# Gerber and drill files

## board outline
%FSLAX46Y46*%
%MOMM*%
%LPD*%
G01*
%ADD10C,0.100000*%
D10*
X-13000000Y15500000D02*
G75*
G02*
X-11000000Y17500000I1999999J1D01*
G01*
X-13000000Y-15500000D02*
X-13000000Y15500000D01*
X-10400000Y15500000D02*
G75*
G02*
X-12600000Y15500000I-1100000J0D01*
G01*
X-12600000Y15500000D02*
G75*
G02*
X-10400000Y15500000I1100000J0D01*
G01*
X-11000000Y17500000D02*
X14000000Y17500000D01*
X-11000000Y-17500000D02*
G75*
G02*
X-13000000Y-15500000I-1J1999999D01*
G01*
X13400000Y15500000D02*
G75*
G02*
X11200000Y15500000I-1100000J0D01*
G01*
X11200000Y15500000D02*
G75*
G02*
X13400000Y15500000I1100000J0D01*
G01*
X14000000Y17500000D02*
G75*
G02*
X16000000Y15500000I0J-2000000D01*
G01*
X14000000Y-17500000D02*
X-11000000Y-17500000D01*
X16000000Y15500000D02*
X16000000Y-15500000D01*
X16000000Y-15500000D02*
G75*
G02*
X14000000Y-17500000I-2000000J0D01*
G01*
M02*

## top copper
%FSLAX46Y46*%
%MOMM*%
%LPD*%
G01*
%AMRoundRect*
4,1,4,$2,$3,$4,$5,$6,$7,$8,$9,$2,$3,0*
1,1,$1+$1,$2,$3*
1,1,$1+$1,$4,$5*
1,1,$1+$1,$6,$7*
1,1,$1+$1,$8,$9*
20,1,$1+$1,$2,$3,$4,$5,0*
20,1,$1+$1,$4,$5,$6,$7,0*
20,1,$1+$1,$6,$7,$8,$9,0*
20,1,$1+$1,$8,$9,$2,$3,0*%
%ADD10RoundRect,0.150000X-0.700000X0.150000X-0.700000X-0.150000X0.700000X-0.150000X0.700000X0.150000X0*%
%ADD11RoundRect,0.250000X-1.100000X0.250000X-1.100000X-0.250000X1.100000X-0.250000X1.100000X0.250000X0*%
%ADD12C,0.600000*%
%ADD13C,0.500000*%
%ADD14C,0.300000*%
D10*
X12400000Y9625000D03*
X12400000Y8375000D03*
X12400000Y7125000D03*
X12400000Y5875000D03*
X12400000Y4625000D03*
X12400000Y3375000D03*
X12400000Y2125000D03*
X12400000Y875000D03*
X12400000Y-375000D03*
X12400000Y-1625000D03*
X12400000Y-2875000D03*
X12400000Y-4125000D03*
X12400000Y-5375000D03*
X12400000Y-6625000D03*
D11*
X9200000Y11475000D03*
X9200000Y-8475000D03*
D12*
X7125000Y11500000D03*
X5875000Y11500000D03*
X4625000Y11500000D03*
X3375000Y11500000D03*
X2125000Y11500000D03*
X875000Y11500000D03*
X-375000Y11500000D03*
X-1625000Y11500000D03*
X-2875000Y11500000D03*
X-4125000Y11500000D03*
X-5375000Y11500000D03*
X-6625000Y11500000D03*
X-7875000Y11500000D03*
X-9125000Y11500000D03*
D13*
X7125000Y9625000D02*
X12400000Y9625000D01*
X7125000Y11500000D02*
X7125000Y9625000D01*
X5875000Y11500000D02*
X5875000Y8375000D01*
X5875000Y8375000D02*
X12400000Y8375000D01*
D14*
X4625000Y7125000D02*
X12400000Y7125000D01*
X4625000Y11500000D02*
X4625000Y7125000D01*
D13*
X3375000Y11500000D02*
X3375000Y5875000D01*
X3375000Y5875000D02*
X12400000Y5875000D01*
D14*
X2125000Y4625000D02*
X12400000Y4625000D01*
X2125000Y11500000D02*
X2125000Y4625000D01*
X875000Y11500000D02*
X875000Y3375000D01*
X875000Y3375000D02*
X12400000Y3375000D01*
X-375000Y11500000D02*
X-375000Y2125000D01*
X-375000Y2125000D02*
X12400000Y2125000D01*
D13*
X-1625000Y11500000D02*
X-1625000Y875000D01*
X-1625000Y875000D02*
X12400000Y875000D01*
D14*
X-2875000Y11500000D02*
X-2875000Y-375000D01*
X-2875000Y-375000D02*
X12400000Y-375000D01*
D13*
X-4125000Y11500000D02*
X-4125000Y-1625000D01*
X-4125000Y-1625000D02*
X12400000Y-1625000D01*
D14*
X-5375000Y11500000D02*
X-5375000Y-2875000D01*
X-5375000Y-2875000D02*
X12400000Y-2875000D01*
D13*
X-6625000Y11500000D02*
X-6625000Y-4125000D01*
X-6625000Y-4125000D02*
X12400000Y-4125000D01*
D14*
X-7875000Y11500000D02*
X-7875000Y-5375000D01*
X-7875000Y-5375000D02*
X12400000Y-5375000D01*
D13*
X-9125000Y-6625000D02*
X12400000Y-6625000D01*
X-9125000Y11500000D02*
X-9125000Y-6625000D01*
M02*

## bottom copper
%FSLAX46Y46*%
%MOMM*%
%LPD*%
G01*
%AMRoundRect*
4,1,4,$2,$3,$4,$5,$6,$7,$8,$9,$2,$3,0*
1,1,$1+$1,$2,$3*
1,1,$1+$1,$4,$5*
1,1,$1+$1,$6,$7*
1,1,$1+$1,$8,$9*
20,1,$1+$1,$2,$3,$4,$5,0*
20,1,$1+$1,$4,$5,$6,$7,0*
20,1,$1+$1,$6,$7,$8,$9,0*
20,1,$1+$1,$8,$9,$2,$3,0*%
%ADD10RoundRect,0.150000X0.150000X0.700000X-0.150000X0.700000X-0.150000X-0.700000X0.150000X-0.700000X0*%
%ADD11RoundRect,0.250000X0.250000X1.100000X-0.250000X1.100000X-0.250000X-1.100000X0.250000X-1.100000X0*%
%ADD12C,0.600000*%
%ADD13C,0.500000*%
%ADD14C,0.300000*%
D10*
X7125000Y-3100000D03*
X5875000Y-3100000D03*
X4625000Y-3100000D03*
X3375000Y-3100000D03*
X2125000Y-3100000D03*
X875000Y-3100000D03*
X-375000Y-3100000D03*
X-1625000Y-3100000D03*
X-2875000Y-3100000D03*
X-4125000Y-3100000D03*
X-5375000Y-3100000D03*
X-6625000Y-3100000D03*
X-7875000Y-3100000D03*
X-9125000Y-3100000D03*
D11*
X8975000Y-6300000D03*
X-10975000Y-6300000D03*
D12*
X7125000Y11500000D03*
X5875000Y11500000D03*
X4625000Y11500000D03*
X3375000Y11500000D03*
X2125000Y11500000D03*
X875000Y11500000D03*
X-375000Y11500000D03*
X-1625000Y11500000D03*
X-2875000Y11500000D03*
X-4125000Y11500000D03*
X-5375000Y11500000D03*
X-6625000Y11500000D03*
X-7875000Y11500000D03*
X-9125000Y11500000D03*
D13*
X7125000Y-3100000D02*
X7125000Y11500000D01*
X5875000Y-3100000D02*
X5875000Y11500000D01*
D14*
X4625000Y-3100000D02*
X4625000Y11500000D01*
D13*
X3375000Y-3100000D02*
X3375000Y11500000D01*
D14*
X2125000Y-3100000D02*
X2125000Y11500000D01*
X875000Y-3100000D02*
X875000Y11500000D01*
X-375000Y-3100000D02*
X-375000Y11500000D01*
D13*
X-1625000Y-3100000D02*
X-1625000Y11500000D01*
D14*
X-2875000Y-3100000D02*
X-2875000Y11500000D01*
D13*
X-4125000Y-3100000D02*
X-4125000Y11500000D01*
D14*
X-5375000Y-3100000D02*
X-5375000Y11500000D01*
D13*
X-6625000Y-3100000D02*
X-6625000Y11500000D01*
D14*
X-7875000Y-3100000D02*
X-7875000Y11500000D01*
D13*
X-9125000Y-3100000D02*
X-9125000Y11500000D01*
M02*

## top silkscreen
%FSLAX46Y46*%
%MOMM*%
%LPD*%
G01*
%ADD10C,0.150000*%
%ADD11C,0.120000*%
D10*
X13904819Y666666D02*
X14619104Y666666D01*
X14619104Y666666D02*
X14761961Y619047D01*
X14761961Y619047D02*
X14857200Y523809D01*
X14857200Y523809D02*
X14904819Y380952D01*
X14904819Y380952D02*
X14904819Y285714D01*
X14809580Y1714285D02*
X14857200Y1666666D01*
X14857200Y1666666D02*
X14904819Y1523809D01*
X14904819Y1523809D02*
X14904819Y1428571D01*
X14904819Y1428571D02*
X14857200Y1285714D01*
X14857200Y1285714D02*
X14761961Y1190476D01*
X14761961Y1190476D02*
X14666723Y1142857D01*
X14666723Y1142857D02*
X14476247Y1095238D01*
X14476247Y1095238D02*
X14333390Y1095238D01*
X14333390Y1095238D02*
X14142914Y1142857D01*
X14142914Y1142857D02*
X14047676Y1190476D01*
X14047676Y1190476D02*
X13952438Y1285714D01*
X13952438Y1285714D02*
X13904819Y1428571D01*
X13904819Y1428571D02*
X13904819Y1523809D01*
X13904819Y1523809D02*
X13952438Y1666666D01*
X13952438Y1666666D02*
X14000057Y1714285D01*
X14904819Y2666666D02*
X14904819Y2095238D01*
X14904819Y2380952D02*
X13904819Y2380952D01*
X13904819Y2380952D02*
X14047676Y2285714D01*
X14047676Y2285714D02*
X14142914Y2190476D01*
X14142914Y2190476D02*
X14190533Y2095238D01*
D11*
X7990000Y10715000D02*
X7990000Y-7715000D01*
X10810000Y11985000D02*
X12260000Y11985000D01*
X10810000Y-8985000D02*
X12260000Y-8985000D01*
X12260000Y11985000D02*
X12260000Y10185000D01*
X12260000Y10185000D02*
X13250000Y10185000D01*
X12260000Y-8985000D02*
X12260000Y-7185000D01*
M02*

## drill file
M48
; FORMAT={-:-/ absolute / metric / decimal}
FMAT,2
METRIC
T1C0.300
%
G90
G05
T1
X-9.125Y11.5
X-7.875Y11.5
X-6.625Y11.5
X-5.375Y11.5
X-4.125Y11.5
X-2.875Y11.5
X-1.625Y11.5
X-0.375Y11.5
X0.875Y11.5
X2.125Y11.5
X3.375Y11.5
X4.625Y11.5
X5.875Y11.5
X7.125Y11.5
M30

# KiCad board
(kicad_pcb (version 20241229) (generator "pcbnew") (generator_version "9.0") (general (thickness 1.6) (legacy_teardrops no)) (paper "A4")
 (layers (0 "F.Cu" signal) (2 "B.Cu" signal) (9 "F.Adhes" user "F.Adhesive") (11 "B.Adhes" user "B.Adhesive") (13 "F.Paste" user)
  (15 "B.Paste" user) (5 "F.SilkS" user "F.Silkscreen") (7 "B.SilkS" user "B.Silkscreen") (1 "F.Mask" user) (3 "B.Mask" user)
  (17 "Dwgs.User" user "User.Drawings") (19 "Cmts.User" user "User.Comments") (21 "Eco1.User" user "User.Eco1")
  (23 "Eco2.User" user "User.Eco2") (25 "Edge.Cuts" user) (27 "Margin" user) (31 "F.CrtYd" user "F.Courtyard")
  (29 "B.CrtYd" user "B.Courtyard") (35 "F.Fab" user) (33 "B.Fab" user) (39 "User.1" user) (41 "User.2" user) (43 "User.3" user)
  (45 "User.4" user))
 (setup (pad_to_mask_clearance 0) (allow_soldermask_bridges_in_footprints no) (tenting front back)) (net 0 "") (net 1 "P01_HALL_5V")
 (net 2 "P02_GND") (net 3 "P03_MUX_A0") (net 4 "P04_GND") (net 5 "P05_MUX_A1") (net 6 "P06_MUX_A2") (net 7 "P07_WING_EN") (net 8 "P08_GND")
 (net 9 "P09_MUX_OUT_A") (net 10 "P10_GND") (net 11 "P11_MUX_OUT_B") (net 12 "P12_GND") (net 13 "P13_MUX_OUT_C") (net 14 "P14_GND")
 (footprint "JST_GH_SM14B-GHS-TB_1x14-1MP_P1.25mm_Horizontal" (layer "F.Cu") (at 10.55 -1.5 -90)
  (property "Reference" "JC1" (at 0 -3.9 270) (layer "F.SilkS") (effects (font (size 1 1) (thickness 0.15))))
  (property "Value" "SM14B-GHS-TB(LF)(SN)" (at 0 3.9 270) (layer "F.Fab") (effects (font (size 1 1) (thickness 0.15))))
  (fp_line (start -9.215 2.56) (end 9.215 2.56) (stroke (width 0.12) (type solid)) (layer "F.SilkS"))
  (fp_line (start -10.485 -0.26) (end -10.485 -1.71) (stroke (width 0.12) (type solid)) (layer "F.SilkS"))
  (fp_line (start 10.485 -0.26) (end 10.485 -1.71) (stroke (width 0.12) (type solid)) (layer "F.SilkS"))
  (fp_line (start -10.485 -1.71) (end -8.685 -1.71) (stroke (width 0.12) (type solid)) (layer "F.SilkS"))
  (fp_line (start -8.685 -1.71) (end -8.685 -2.7) (stroke (width 0.12) (type solid)) (layer "F.SilkS"))
  (fp_line (start 10.485 -1.71) (end 8.685 -1.71) (stroke (width 0.12) (type solid)) (layer "F.SilkS"))
  (pad "1" smd roundrect (at -8.125 -1.85 270) (size 0.6 1.7) (layers "F.Cu" "F.Mask" "F.Paste") (roundrect_rratio 0.25)
   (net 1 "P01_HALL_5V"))
  (pad "2" smd roundrect (at -6.875 -1.85 270) (size 0.6 1.7) (layers "F.Cu" "F.Mask" "F.Paste") (roundrect_rratio 0.25) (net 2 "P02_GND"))
  (pad "3" smd roundrect (at -5.625 -1.85 270) (size 0.6 1.7) (layers "F.Cu" "F.Mask" "F.Paste") (roundrect_rratio 0.25)
   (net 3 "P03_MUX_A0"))
  (pad "4" smd roundrect (at -4.375 -1.85 270) (size 0.6 1.7) (layers "F.Cu" "F.Mask" "F.Paste") (roundrect_rratio 0.25) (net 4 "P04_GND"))
  (pad "5" smd roundrect (at -3.125 -1.85 270) (size 0.6 1.7) (layers "F.Cu" "F.Mask" "F.Paste") (roundrect_rratio 0.25)
   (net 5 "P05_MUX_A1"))
  (pad "6" smd roundrect (at -1.875 -1.85 270) (size 0.6 1.7) (layers "F.Cu" "F.Mask" "F.Paste") (roundrect_rratio 0.25)
   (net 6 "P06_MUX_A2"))
  (pad "7" smd roundrect (at -0.625 -1.85 270) (size 0.6 1.7) (layers "F.Cu" "F.Mask" "F.Paste") (roundrect_rratio 0.25)
   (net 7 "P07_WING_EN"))
  (pad "8" smd roundrect (at 0.625 -1.85 270) (size 0.6 1.7) (layers "F.Cu" "F.Mask" "F.Paste") (roundrect_rratio 0.25) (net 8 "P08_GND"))
  (pad "9" smd roundrect (at 1.875 -1.85 270) (size 0.6 1.7) (layers "F.Cu" "F.Mask" "F.Paste") (roundrect_rratio 0.25)
   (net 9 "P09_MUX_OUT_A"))
  (pad "10" smd roundrect (at 3.125 -1.85 270) (size 0.6 1.7) (layers "F.Cu" "F.Mask" "F.Paste") (roundrect_rratio 0.25) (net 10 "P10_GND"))
  (pad "11" smd roundrect (at 4.375 -1.85 270) (size 0.6 1.7) (layers "F.Cu" "F.Mask" "F.Paste") (roundrect_rratio 0.25)
   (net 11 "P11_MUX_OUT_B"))
  (pad "12" smd roundrect (at 5.625 -1.85 270) (size 0.6 1.7) (layers "F.Cu" "F.Mask" "F.Paste") (roundrect_rratio 0.25) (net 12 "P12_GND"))
  (pad "13" smd roundrect (at 6.875 -1.85 270) (size 0.6 1.7) (layers "F.Cu" "F.Mask" "F.Paste") (roundrect_rratio 0.25)
   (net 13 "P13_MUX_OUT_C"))
  (pad "14" smd roundrect (at 8.125 -1.85 270) (size 0.6 1.7) (layers "F.Cu" "F.Mask" "F.Paste") (roundrect_rratio 0.25) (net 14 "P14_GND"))
  (pad "15" smd roundrect (at -9.975 1.35 270) (size 1 2.7) (layers "F.Cu" "F.Mask" "F.Paste") (roundrect_rratio 0.25))
  (pad "15" smd roundrect (at 9.975 1.35 270) (size 1 2.7) (layers "F.Cu" "F.Mask" "F.Paste") (roundrect_rratio 0.25)))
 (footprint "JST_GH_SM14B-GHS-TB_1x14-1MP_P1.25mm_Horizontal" (layer "B.Cu") (at -1 4.95 180)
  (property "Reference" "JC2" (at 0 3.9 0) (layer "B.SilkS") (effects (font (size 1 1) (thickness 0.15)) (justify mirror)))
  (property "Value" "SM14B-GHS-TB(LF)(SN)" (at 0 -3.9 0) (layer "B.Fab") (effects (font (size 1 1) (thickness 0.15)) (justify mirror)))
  (pad "1" smd roundrect (at -8.125 1.85 180) (size 0.6 1.7) (layers "B.Cu" "B.Mask" "B.Paste") (roundrect_rratio 0.25)
   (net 1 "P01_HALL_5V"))
  (pad "2" smd roundrect (at -6.875 1.85 180) (size 0.6 1.7) (layers "B.Cu" "B.Mask" "B.Paste") (roundrect_rratio 0.25) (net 2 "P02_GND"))
  (pad "3" smd roundrect (at -5.625 1.85 180) (size 0.6 1.7) (layers "B.Cu" "B.Mask" "B.Paste") (roundrect_rratio 0.25) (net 3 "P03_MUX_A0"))
  (pad "4" smd roundrect (at -4.375 1.85 180) (size 0.6 1.7) (layers "B.Cu" "B.Mask" "B.Paste") (roundrect_rratio 0.25) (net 4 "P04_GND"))
  (pad "5" smd roundrect (at -3.125 1.85 180) (size 0.6 1.7) (layers "B.Cu" "B.Mask" "B.Paste") (roundrect_rratio 0.25) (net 5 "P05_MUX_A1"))
  (pad "6" smd roundrect (at -1.875 1.85 180) (size 0.6 1.7) (layers "B.Cu" "B.Mask" "B.Paste") (roundrect_rratio 0.25) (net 6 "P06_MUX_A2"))
  (pad "7" smd roundrect (at -0.625 1.85 180) (size 0.6 1.7) (layers "B.Cu" "B.Mask" "B.Paste") (roundrect_rratio 0.25)
   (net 7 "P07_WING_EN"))
  (pad "8" smd roundrect (at 0.625 1.85 180) (size 0.6 1.7) (layers "B.Cu" "B.Mask" "B.Paste") (roundrect_rratio 0.25) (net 8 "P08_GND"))
  (pad "9" smd roundrect (at 1.875 1.85 180) (size 0.6 1.7) (layers "B.Cu" "B.Mask" "B.Paste") (roundrect_rratio 0.25)
   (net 9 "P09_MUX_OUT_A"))
  (pad "10" smd roundrect (at 3.125 1.85 180) (size 0.6 1.7) (layers "B.Cu" "B.Mask" "B.Paste") (roundrect_rratio 0.25) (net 10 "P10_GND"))
  (pad "11" smd roundrect (at 4.375 1.85 180) (size 0.6 1.7) (layers "B.Cu" "B.Mask" "B.Paste") (roundrect_rratio 0.25)
   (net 11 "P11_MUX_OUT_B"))
  (pad "12" smd roundrect (at 5.625 1.85 180) (size 0.6 1.7) (layers "B.Cu" "B.Mask" "B.Paste") (roundrect_rratio 0.25) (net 12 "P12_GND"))
  (pad "13" smd roundrect (at 6.875 1.85 180) (size 0.6 1.7) (layers "B.Cu" "B.Mask" "B.Paste") (roundrect_rratio 0.25)
   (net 13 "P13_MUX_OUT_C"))
  (pad "14" smd roundrect (at 8.125 1.85 180) (size 0.6 1.7) (layers "B.Cu" "B.Mask" "B.Paste") (roundrect_rratio 0.25) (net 14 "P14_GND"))
  (pad "15" smd roundrect (at -9.975 -1.35 180) (size 1 2.7) (layers "B.Cu" "B.Mask" "B.Paste") (roundrect_rratio 0.25))
  (pad "15" smd roundrect (at 9.975 -1.35 180) (size 1 2.7) (layers "B.Cu" "B.Mask" "B.Paste") (roundrect_rratio 0.25)))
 (gr_arc (start -13 -15.5) (mid -12.414214 -16.914214) (end -11 -17.5) (stroke (width 0.1) (type default)) (layer "Edge.Cuts"))
 (gr_line (start -13 15.5) (end -13 -15.5) (stroke (width 0.1) (type default)) (layer "Edge.Cuts"))
 (gr_circle (center -11.5 -15.5) (end -10.4 -15.5) (stroke (width 0.1) (type default)) (fill no) (layer "Edge.Cuts"))
 (gr_line (start -11 -17.5) (end 14 -17.5) (stroke (width 0.1) (type default)) (layer "Edge.Cuts"))
 (gr_arc (start -11 17.5) (mid -12.414214 16.914214) (end -13 15.5) (stroke (width 0.1) (type default)) (layer "Edge.Cuts"))
 (gr_circle (center 12.3 -15.5) (end 13.4 -15.5) (stroke (width 0.1) (type default)) (fill no) (layer "Edge.Cuts"))
 (gr_arc (start 14 -17.5) (mid 15.414214 -16.914214) (end 16 -15.5) (stroke (width 0.1) (type default)) (layer "Edge.Cuts"))
 (gr_line (start 14 17.5) (end -11 17.5) (stroke (width 0.1) (type default)) (layer "Edge.Cuts"))
 (gr_line (start 16 -15.5) (end 16 15.5) (stroke (width 0.1) (type default)) (layer "Edge.Cuts"))
 (gr_arc (start 16 15.5) (mid 15.414214 16.914214) (end 14 17.5) (stroke (width 0.1) (type default)) (layer "Edge.Cuts"))
 (segment (start 7.125 -9.625) (end 12.4 -9.625) (width 0.5) (layer "F.Cu") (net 1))
 (segment (start 7.125 -11.5) (end 7.125 -9.625) (width 0.5) (layer "F.Cu") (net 1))
 (via (at 7.125 -11.5) (size 0.6) (drill 0.3) (layers "F.Cu" "B.Cu") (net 1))
 (segment (start 7.125 3.1) (end 7.125 -11.5) (width 0.5) (layer "B.Cu") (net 1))
 (segment (start 5.875 -11.5) (end 5.875 -8.375) (width 0.5) (layer "F.Cu") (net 2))
 (segment (start 5.875 -8.375) (end 12.4 -8.375) (width 0.5) (layer "F.Cu") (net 2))
 (via (at 5.875 -11.5) (size 0.6) (drill 0.3) (layers "F.Cu" "B.Cu") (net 2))
 (segment (start 5.875 3.1) (end 5.875 -11.5) (width 0.5) (layer "B.Cu") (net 2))
 (segment (start 4.625 -7.125) (end 12.4 -7.125) (width 0.3) (layer "F.Cu") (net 3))
 (segment (start 4.625 -11.5) (end 4.625 -7.125) (width 0.3) (layer "F.Cu") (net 3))
 (via (at 4.625 -11.5) (size 0.6) (drill 0.3) (layers "F.Cu" "B.Cu") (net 3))
 (segment (start 4.625 3.1) (end 4.625 -11.5) (width 0.3) (layer "B.Cu") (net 3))
 (segment (start 3.375 -11.5) (end 3.375 -5.875) (width 0.5) (layer "F.Cu") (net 4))
 (segment (start 3.375 -5.875) (end 12.4 -5.875) (width 0.5) (layer "F.Cu") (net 4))
 (via (at 3.375 -11.5) (size 0.6) (drill 0.3) (layers "F.Cu" "B.Cu") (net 4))
 (segment (start 3.375 3.1) (end 3.375 -11.5) (width 0.5) (layer "B.Cu") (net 4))
 (segment (start 2.125 -4.625) (end 12.4 -4.625) (width 0.3) (layer "F.Cu") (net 5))
 (segment (start 2.125 -11.5) (end 2.125 -4.625) (width 0.3) (layer "F.Cu") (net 5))
 (via (at 2.125 -11.5) (size 0.6) (drill 0.3) (layers "F.Cu" "B.Cu") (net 5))
 (segment (start 2.125 3.1) (end 2.125 -11.5) (width 0.3) (layer "B.Cu") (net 5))
 (segment (start 0.875 -11.5) (end 0.875 -3.375) (width 0.3) (layer "F.Cu") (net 6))
 (segment (start 0.875 -3.375) (end 12.4 -3.375) (width 0.3) (layer "F.Cu") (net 6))
 (via (at 0.875 -11.5) (size 0.6) (drill 0.3) (layers "F.Cu" "B.Cu") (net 6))
 (segment (start 0.875 3.1) (end 0.875 -11.5) (width 0.3) (layer "B.Cu") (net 6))
 (segment (start -0.375 -11.5) (end -0.375 -2.125) (width 0.3) (layer "F.Cu") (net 7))
 (segment (start -0.375 -2.125) (end 12.4 -2.125) (width 0.3) (layer "F.Cu") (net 7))
 (via (at -0.375 -11.5) (size 0.6) (drill 0.3) (layers "F.Cu" "B.Cu") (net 7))
 (segment (start -0.375 3.1) (end -0.375 -11.5) (width 0.3) (layer "B.Cu") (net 7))
 (segment (start -1.625 -11.5) (end -1.625 -0.875) (width 0.5) (layer "F.Cu") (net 8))
 (segment (start -1.625 -0.875) (end 12.4 -0.875) (width 0.5) (layer "F.Cu") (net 8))
 (via (at -1.625 -11.5) (size 0.6) (drill 0.3) (layers "F.Cu" "B.Cu") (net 8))
 (segment (start -1.625 3.1) (end -1.625 -11.5) (width 0.5) (layer "B.Cu") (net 8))
 (segment (start -2.875 -11.5) (end -2.875 0.375) (width 0.3) (layer "F.Cu") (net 9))
 (segment (start -2.875 0.375) (end 12.4 0.375) (width 0.3) (layer "F.Cu") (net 9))
 (via (at -2.875 -11.5) (size 0.6) (drill 0.3) (layers "F.Cu" "B.Cu") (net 9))
 (segment (start -2.875 3.1) (end -2.875 -11.5) (width 0.3) (layer "B.Cu") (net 9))
 (segment (start -4.125 -11.5) (end -4.125 1.625) (width 0.5) (layer "F.Cu") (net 10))
 (segment (start -4.125 1.625) (end 12.4 1.625) (width 0.5) (layer "F.Cu") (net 10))
 (via (at -4.125 -11.5) (size 0.6) (drill 0.3) (layers "F.Cu" "B.Cu") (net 10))
 (segment (start -4.125 3.1) (end -4.125 -11.5) (width 0.5) (layer "B.Cu") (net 10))
 (segment (start -5.375 -11.5) (end -5.375 2.875) (width 0.3) (layer "F.Cu") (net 11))
 (segment (start -5.375 2.875) (end 12.4 2.875) (width 0.3) (layer "F.Cu") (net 11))
 (via (at -5.375 -11.5) (size 0.6) (drill 0.3) (layers "F.Cu" "B.Cu") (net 11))
 (segment (start -5.375 3.1) (end -5.375 -11.5) (width 0.3) (layer "B.Cu") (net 11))
 (segment (start -6.625 -11.5) (end -6.625 4.125) (width 0.5) (layer "F.Cu") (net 12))
 (segment (start -6.625 4.125) (end 12.4 4.125) (width 0.5) (layer "F.Cu") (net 12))
 (via (at -6.625 -11.5) (size 0.6) (drill 0.3) (layers "F.Cu" "B.Cu") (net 12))
 (segment (start -6.625 3.1) (end -6.625 -11.5) (width 0.5) (layer "B.Cu") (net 12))
 (segment (start -7.875 -11.5) (end -7.875 5.375) (width 0.3) (layer "F.Cu") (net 13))
 (segment (start -7.875 5.375) (end 12.4 5.375) (width 0.3) (layer "F.Cu") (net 13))
 (via (at -7.875 -11.5) (size 0.6) (drill 0.3) (layers "F.Cu" "B.Cu") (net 13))
 (segment (start -7.875 3.1) (end -7.875 -11.5) (width 0.3) (layer "B.Cu") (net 13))
 (segment (start -9.125 6.625) (end 12.4 6.625) (width 0.5) (layer "F.Cu") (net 14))
 (segment (start -9.125 -11.5) (end -9.125 6.625) (width 0.5) (layer "F.Cu") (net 14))
 (via (at -9.125 -11.5) (size 0.6) (drill 0.3) (layers "F.Cu" "B.Cu") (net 14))
 (segment (start -9.125 3.1) (end -9.125 -11.5) (width 0.5) (layer "B.Cu") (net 14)))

